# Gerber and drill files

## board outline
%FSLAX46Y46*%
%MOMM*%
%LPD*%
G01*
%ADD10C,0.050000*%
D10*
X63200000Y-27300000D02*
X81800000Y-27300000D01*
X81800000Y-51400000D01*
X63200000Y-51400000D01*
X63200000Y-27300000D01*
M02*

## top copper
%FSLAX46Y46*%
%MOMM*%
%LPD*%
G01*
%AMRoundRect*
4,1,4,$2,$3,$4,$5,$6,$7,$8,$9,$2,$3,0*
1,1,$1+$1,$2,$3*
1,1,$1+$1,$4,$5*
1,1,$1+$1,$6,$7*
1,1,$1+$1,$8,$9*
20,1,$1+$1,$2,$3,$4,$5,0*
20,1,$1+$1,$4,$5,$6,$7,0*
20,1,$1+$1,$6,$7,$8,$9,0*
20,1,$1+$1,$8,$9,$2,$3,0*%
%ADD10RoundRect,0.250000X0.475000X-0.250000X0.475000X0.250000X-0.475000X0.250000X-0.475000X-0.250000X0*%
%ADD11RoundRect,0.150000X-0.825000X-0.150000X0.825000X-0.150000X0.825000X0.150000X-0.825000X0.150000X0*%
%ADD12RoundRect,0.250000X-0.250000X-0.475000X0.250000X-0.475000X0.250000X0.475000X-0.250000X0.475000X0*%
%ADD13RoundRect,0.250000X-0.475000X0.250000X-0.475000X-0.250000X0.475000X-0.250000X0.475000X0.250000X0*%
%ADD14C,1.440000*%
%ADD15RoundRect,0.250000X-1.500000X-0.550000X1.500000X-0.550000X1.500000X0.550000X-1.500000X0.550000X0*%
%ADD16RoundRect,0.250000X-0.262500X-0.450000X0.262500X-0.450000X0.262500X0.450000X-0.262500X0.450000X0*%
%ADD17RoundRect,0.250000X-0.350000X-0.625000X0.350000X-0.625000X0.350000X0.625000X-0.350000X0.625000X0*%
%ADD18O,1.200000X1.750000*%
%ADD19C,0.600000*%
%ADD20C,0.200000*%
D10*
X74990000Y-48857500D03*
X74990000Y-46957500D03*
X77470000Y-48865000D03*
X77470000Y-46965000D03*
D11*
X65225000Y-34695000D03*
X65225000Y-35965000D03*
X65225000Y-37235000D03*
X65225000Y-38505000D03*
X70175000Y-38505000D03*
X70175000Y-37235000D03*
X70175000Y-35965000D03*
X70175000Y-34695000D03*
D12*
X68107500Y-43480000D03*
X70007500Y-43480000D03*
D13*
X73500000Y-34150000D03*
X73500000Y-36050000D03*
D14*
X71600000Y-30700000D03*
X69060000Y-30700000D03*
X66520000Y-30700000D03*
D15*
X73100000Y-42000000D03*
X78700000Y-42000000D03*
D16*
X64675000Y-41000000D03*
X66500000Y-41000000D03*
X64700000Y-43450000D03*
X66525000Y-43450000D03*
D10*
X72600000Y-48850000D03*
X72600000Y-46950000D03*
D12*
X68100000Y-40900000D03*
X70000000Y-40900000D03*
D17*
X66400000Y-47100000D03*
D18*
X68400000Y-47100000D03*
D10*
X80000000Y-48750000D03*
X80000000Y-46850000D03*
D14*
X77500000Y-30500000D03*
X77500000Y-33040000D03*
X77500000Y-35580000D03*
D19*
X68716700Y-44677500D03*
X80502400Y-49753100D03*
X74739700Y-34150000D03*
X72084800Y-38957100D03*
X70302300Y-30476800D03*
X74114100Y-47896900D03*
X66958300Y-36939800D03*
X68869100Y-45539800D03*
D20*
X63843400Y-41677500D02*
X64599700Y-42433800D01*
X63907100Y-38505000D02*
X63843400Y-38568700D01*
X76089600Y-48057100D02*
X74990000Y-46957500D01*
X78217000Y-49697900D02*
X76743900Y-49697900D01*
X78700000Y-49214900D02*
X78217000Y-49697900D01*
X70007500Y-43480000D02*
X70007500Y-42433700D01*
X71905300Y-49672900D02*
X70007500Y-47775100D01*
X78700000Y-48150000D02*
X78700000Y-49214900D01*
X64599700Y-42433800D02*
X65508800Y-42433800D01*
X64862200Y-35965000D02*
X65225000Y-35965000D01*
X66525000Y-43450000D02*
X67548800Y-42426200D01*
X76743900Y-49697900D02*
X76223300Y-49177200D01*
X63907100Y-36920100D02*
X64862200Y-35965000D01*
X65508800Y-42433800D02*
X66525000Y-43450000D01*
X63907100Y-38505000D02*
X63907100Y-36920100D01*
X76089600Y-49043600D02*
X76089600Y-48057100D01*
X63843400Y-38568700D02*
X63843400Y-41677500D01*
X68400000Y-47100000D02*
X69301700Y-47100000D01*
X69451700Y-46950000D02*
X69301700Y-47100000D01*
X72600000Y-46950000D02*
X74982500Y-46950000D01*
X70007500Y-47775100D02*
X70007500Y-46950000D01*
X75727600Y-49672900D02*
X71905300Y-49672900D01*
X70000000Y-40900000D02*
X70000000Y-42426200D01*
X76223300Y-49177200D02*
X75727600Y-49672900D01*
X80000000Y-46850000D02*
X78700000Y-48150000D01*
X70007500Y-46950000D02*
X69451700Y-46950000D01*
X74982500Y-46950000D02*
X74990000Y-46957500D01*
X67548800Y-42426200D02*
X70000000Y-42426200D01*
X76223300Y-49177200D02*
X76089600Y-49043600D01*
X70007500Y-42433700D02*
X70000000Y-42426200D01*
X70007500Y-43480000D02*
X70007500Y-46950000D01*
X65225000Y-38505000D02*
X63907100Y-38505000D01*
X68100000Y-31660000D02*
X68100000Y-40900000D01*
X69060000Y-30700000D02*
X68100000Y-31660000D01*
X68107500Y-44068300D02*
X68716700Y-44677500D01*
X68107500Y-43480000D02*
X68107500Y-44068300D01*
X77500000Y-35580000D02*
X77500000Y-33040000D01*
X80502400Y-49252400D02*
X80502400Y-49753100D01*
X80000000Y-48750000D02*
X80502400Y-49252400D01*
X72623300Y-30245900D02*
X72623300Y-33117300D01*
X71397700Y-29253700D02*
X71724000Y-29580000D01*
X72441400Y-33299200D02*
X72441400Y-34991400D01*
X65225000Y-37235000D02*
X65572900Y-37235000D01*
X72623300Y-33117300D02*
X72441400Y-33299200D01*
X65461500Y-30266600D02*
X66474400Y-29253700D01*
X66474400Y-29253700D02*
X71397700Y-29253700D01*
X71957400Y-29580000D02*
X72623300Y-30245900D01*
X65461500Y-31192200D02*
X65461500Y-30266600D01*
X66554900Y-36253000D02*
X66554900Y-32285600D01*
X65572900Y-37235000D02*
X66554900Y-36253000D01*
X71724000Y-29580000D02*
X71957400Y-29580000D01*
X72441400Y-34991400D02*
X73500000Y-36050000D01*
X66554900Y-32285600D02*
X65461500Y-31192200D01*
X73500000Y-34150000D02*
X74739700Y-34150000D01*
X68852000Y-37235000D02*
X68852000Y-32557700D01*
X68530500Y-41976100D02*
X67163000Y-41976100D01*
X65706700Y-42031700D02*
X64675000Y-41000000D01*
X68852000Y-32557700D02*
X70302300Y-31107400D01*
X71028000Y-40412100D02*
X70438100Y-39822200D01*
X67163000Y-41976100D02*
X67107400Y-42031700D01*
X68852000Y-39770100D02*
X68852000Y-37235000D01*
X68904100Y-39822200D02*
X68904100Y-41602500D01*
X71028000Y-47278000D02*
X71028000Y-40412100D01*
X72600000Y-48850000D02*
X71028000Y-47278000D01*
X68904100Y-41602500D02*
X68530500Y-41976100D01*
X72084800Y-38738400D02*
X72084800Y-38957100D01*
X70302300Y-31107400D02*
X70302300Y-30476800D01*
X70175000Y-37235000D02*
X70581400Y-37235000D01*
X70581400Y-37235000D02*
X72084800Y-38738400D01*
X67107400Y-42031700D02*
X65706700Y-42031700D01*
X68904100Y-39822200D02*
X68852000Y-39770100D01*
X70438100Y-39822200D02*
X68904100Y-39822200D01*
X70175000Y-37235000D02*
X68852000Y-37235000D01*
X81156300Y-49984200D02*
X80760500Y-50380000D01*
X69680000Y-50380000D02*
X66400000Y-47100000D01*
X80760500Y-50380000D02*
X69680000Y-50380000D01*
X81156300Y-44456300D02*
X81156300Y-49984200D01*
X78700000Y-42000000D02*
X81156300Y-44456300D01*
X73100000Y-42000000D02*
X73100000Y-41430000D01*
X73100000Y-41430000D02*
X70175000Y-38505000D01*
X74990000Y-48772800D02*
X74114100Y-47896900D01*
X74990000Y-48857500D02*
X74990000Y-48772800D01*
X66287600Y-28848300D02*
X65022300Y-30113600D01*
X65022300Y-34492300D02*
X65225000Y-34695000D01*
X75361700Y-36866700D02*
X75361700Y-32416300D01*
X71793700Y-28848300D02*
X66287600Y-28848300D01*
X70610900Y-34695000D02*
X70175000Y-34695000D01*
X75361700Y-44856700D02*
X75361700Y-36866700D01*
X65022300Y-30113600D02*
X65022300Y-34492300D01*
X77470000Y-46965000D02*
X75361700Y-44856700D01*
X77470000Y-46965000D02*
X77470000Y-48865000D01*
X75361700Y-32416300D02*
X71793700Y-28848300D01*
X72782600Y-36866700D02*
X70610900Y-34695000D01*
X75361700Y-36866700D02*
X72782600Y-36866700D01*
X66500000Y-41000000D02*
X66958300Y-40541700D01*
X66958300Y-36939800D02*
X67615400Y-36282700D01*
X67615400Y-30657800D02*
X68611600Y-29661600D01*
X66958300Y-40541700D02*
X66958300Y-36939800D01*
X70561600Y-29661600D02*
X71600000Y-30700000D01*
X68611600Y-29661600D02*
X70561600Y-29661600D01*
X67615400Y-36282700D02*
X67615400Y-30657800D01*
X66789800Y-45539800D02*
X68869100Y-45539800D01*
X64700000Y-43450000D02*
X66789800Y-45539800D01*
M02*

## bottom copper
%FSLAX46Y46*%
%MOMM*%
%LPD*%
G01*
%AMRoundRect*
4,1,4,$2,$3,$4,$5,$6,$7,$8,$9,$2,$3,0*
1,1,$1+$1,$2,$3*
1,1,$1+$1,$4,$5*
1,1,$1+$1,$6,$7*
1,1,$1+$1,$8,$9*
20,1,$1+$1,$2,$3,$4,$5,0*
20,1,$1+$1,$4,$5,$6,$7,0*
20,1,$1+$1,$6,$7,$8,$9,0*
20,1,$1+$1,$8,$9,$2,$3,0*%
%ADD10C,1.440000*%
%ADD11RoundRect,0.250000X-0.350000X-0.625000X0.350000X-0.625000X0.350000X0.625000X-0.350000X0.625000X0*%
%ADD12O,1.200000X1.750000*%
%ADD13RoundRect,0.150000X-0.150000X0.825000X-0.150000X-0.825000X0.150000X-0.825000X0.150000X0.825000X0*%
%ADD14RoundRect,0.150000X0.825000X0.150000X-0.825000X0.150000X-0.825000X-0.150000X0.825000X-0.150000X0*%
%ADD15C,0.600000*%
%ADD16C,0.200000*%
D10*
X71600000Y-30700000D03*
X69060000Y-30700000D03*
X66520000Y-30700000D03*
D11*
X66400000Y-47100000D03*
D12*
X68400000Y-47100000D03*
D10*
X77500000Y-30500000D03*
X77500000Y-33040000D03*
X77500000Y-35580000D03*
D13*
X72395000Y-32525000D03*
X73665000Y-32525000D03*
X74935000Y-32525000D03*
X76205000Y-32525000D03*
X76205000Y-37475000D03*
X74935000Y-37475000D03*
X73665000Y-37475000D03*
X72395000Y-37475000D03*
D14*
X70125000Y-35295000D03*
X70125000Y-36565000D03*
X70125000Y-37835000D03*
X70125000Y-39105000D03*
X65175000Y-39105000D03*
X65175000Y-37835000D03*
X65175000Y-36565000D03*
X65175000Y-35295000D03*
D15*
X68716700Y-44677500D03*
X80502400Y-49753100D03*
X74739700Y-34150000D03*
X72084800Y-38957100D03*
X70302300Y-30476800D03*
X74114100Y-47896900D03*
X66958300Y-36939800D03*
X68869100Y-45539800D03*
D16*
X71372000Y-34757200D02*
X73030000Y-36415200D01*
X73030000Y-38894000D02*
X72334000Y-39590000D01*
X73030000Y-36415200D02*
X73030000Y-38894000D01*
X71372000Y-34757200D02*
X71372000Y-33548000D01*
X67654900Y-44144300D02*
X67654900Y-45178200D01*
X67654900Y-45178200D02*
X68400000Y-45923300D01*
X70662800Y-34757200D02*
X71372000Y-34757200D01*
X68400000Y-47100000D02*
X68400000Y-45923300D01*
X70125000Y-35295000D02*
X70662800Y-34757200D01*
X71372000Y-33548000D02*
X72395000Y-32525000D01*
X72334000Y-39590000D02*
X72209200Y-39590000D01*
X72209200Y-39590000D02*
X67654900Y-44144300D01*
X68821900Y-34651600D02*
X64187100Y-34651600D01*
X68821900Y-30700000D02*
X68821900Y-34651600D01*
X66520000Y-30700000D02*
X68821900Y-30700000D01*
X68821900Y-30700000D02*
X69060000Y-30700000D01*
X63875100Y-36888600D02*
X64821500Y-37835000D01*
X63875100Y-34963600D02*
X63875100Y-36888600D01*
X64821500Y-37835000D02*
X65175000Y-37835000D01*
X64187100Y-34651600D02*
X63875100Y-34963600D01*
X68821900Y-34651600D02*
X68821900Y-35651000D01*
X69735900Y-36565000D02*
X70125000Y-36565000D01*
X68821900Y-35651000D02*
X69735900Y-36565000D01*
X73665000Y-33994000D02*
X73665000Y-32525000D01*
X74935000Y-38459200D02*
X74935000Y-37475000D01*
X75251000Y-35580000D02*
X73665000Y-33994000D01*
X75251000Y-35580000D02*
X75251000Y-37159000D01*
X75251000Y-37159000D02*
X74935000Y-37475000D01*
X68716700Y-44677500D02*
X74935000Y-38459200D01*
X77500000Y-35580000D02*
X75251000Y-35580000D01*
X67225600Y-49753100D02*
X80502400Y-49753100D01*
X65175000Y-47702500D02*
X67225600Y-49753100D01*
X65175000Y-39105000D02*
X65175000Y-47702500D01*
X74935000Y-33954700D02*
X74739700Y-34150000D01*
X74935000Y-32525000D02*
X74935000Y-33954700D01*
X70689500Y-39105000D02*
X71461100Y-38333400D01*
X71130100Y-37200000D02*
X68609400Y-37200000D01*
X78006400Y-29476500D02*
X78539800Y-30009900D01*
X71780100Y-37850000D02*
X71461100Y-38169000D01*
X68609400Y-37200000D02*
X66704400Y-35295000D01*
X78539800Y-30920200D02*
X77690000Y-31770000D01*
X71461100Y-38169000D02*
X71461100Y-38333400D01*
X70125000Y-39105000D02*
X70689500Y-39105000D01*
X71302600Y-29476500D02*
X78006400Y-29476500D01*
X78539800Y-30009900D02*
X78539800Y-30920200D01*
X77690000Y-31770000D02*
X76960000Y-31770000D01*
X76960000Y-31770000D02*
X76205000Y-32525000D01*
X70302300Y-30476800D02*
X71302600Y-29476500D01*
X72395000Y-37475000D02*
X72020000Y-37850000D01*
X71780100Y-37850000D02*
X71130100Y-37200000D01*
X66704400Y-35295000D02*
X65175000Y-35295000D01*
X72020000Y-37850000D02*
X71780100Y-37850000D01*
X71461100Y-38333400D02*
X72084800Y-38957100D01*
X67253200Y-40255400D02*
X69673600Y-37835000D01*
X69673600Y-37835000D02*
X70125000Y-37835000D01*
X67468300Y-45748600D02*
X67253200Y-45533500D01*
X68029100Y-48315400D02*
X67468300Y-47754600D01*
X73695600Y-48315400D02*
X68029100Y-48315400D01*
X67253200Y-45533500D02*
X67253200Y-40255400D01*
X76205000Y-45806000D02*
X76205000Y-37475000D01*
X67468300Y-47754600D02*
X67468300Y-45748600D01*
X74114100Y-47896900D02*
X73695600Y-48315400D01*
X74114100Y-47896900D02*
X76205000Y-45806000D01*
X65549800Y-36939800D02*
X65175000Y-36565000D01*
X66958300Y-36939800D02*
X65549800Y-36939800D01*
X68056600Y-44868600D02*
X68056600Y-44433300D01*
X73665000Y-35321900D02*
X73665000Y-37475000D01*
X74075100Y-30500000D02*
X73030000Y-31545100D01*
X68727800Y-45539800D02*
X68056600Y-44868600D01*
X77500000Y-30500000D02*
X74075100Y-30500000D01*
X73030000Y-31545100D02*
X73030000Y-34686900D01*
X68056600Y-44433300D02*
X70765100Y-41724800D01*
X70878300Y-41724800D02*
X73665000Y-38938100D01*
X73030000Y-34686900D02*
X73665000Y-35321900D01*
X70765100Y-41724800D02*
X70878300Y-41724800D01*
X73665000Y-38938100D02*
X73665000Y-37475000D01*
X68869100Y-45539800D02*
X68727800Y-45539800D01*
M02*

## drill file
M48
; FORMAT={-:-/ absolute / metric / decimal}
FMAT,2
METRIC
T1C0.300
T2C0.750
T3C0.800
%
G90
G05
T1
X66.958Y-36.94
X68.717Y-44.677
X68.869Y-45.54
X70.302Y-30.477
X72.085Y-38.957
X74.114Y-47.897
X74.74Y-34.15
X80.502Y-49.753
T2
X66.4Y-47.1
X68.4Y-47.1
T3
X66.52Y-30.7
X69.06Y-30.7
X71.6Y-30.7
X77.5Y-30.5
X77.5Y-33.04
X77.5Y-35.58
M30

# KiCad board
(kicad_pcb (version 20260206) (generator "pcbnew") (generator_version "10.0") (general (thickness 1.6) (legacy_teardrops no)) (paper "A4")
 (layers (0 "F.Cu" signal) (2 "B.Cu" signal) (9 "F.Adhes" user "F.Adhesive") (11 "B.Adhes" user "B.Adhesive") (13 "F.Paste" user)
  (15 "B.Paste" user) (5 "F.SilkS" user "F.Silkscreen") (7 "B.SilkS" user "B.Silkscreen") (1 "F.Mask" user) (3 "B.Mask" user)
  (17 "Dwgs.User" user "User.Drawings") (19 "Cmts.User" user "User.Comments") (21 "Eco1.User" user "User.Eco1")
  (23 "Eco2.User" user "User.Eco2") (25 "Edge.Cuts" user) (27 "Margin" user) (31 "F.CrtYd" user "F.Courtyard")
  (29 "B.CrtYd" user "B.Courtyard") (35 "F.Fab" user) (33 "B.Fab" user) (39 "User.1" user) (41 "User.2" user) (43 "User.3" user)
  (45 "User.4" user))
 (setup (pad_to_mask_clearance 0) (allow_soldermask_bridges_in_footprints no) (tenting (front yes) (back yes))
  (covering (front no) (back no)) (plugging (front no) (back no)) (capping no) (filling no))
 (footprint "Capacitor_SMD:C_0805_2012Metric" (layer "F.Cu") (at 74.99 47.9075 90)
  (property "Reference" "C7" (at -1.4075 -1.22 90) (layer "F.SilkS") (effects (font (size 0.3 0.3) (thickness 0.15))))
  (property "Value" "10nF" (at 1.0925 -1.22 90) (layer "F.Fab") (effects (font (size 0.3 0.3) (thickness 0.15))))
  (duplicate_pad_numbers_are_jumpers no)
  (pad "1" smd roundrect (at -0.95 0 90) (size 1 1.45) (layers "F.Cu" "F.Mask" "F.Paste") (roundrect_rratio 0.25) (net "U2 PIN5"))
  (pad "2" smd roundrect (at 0.95 0 90) (size 1 1.45) (layers "F.Cu" "F.Mask" "F.Paste") (roundrect_rratio 0.25) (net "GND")))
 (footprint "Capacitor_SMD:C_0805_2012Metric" (layer "F.Cu") (at 77.47 47.915 90)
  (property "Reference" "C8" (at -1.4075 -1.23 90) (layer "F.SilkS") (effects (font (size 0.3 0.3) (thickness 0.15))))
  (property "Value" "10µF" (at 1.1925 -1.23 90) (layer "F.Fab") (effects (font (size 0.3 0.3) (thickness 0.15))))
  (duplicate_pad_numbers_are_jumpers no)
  (pad "1" smd roundrect (at -0.95 0 90) (size 1 1.45) (layers "F.Cu" "F.Mask" "F.Paste") (roundrect_rratio 0.25) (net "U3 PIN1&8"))
  (pad "2" smd roundrect (at 0.95 0 90) (size 1 1.45) (layers "F.Cu" "F.Mask" "F.Paste") (roundrect_rratio 0.25) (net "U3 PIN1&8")))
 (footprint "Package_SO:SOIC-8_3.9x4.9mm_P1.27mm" (layer "F.Cu") (at 67.7 36.6)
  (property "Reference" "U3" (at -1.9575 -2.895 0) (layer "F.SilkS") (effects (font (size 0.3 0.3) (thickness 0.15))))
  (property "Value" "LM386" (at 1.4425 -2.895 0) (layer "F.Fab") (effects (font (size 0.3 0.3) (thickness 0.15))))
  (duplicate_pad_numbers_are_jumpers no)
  (pad "1" smd roundrect (at -2.475 -1.905) (size 1.95 0.6) (layers "F.Cu" "F.Mask" "F.Paste") (roundrect_rratio 0.25) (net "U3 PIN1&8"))
  (pad "2" smd roundrect (at -2.475 -0.635) (size 1.95 0.6) (layers "F.Cu" "F.Mask" "F.Paste") (roundrect_rratio 0.25) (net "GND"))
  (pad "3" smd roundrect (at -2.475 0.635) (size 1.95 0.6) (layers "F.Cu" "F.Mask" "F.Paste") (roundrect_rratio 0.25) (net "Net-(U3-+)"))
  (pad "4" smd roundrect (at -2.475 1.905) (size 1.95 0.6) (layers "F.Cu" "F.Mask" "F.Paste") (roundrect_rratio 0.25) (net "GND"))
  (pad "5" smd roundrect (at 2.475 1.905) (size 1.95 0.6) (layers "F.Cu" "F.Mask" "F.Paste") (roundrect_rratio 0.25) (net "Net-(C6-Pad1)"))
  (pad "6" smd roundrect (at 2.475 0.635) (size 1.95 0.6) (layers "F.Cu" "F.Mask" "F.Paste") (roundrect_rratio 0.25) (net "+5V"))
  (pad "7" smd roundrect (at 2.475 -0.635) (size 1.95 0.6) (layers "F.Cu" "F.Mask" "F.Paste") (roundrect_rratio 0.25)
   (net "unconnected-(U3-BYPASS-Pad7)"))
  (pad "8" smd roundrect (at 2.475 -1.905) (size 1.95 0.6) (layers "F.Cu" "F.Mask" "F.Paste") (roundrect_rratio 0.25) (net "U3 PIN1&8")))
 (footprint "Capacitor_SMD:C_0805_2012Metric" (layer "F.Cu") (at 69.0575 43.48)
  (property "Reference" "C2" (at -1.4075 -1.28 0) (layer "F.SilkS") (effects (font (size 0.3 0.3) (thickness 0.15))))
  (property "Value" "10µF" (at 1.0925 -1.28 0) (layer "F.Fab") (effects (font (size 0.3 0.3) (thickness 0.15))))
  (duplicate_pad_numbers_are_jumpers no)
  (pad "1" smd roundrect (at -0.95 0) (size 1 1.45) (layers "F.Cu" "F.Mask" "F.Paste") (roundrect_rratio 0.25) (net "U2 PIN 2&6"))
  (pad "2" smd roundrect (at 0.95 0) (size 1 1.45) (layers "F.Cu" "F.Mask" "F.Paste") (roundrect_rratio 0.25) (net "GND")))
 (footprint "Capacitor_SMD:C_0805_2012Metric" (layer "F.Cu") (at 73.5 35.1 -90)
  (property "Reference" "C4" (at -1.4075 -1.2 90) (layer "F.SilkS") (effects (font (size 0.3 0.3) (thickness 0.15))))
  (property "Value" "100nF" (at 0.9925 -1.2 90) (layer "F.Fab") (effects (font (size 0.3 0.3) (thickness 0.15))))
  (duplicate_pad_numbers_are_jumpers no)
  (pad "1" smd roundrect (at -0.95 0 270) (size 1 1.45) (layers "F.Cu" "F.Mask" "F.Paste") (roundrect_rratio 0.25) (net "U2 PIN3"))
  (pad "2" smd roundrect (at 0.95 0 270) (size 1 1.45) (layers "F.Cu" "F.Mask" "F.Paste") (roundrect_rratio 0.25) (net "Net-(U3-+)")))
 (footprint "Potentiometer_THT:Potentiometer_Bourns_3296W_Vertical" (layer "F.Cu") (at 71.6 30.7)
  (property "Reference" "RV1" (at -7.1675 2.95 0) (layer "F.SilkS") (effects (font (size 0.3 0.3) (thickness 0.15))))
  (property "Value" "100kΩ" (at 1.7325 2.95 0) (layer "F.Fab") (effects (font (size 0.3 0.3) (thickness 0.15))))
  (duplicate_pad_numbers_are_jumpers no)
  (pad "1" thru_hole circle (at 0 0) (size 1.44 1.44) (drill 0.8) (layers "*.Cu" "*.Mask") (remove_unused_layers no) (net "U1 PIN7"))
  (pad "2" thru_hole circle (at -2.54 0) (size 1.44 1.44) (drill 0.8) (layers "*.Cu" "*.Mask") (remove_unused_layers no) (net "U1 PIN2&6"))
  (pad "3" thru_hole circle (at -5.08 0) (size 1.44 1.44) (drill 0.8) (layers "*.Cu" "*.Mask") (remove_unused_layers no) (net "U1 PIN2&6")))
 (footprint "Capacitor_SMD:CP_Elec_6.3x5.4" (layer "F.Cu") (at 75.9 42)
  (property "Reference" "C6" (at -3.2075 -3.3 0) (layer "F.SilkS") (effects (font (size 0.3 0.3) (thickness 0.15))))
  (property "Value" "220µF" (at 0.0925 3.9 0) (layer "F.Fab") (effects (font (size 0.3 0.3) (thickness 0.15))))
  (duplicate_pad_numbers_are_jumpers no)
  (pad "1" smd roundrect (at -2.8 0) (size 3.5 1.6) (layers "F.Cu" "F.Mask" "F.Paste") (roundrect_rratio 0.15625) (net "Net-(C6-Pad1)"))
  (pad "2" smd roundrect (at 2.8 0) (size 3.5 1.6) (layers "F.Cu" "F.Mask" "F.Paste") (roundrect_rratio 0.15625) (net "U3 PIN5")))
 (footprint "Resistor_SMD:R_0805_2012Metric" (layer "F.Cu") (at 65.5875 41)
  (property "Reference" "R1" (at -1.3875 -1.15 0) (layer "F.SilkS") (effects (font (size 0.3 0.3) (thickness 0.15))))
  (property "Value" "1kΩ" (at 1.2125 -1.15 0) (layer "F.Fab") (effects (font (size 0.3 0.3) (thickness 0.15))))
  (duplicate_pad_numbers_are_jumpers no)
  (pad "1" smd roundrect (at -0.9125 0) (size 1.025 1.4) (layers "F.Cu" "F.Mask" "F.Paste") (roundrect_rratio 0.243902) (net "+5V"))
  (pad "2" smd roundrect (at 0.9125 0) (size 1.025 1.4) (layers "F.Cu" "F.Mask" "F.Paste") (roundrect_rratio 0.243902) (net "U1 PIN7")))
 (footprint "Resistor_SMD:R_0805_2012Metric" (layer "F.Cu") (at 65.6125 43.45)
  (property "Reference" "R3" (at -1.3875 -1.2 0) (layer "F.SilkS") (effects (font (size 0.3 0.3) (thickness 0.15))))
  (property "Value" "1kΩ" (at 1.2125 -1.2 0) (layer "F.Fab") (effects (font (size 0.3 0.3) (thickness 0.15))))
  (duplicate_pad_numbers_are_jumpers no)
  (pad "1" smd roundrect (at -0.9125 0) (size 1.025 1.4) (layers "F.Cu" "F.Mask" "F.Paste") (roundrect_rratio 0.243902) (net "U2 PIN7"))
  (pad "2" smd roundrect (at 0.9125 0) (size 1.025 1.4) (layers "F.Cu" "F.Mask" "F.Paste") (roundrect_rratio 0.243902) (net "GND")))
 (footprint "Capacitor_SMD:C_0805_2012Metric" (layer "F.Cu") (at 72.6 47.9 90)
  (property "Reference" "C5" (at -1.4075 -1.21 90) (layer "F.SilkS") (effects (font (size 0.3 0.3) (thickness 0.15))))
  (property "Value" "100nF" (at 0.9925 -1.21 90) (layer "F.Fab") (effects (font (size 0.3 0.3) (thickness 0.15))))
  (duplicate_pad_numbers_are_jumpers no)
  (pad "1" smd roundrect (at -0.95 0 90) (size 1 1.45) (layers "F.Cu" "F.Mask" "F.Paste") (roundrect_rratio 0.25) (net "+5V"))
  (pad "2" smd roundrect (at 0.95 0 90) (size 1 1.45) (layers "F.Cu" "F.Mask" "F.Paste") (roundrect_rratio 0.25) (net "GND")))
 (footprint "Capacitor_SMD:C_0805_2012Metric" (layer "F.Cu") (at 69.05 40.9)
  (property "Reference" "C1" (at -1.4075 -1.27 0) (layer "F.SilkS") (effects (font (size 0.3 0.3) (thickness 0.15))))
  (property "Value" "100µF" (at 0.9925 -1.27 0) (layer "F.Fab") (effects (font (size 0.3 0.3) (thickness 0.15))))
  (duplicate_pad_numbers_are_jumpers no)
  (pad "1" smd roundrect (at -0.95 0) (size 1 1.45) (layers "F.Cu" "F.Mask" "F.Paste") (roundrect_rratio 0.25) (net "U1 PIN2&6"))
  (pad "2" smd roundrect (at 0.95 0) (size 1 1.45) (layers "F.Cu" "F.Mask" "F.Paste") (roundrect_rratio 0.25) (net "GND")))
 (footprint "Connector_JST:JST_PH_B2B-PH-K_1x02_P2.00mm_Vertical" (layer "F.Cu") (at 66.4 47.1)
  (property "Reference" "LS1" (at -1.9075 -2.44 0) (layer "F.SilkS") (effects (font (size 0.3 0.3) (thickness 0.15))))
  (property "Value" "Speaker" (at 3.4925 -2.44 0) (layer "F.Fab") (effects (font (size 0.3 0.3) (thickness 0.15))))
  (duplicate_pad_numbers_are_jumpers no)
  (pad "1" thru_hole roundrect (at 0 0) (size 1.2 1.75) (drill 0.75) (layers "*.Cu" "*.Mask") (remove_unused_layers no)
   (roundrect_rratio 0.208333) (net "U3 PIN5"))
  (pad "2" thru_hole oval (at 2 0) (size 1.2 1.75) (drill 0.75) (layers "*.Cu" "*.Mask") (remove_unused_layers no) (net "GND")))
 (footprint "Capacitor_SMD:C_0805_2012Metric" (layer "F.Cu") (at 80 47.8 90)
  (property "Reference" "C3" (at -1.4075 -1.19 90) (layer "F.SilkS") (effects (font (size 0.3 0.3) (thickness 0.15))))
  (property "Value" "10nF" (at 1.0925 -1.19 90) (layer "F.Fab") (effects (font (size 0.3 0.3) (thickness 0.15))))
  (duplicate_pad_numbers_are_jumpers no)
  (pad "1" smd roundrect (at -0.95 0 90) (size 1 1.45) (layers "F.Cu" "F.Mask" "F.Paste") (roundrect_rratio 0.25) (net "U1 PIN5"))
  (pad "2" smd roundrect (at 0.95 0 90) (size 1 1.45) (layers "F.Cu" "F.Mask" "F.Paste") (roundrect_rratio 0.25) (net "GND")))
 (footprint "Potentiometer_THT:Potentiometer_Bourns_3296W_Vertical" (layer "F.Cu") (at 77.5 30.5 90)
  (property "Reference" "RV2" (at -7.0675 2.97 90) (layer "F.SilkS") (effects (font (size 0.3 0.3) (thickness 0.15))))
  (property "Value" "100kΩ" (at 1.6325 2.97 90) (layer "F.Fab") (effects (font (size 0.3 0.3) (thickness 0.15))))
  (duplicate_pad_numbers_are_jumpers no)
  (pad "1" thru_hole circle (at 0 0 90) (size 1.44 1.44) (drill 0.8) (layers "*.Cu" "*.Mask") (remove_unused_layers no) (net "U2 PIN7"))
  (pad "2" thru_hole circle (at -2.54 0 90) (size 1.44 1.44) (drill 0.8) (layers "*.Cu" "*.Mask") (remove_unused_layers no)
   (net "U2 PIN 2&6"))
  (pad "3" thru_hole circle (at -5.08 0 90) (size 1.44 1.44) (drill 0.8) (layers "*.Cu" "*.Mask") (remove_unused_layers no)
   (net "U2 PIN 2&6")))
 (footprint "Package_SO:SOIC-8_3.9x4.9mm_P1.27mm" (layer "B.Cu") (at 74.3 35 -90)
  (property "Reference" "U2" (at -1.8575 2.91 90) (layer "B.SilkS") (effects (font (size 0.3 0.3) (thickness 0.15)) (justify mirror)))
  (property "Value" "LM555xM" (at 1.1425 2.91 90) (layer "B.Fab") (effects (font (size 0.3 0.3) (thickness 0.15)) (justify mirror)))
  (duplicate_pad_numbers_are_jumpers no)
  (pad "1" smd roundrect (at -2.475 1.905 270) (size 1.95 0.6) (layers "B.Cu" "B.Mask" "B.Paste") (roundrect_rratio 0.25) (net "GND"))
  (pad "2" smd roundrect (at -2.475 0.635 270) (size 1.95 0.6) (layers "B.Cu" "B.Mask" "B.Paste") (roundrect_rratio 0.25) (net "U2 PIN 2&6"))
  (pad "3" smd roundrect (at -2.475 -0.635 270) (size 1.95 0.6) (layers "B.Cu" "B.Mask" "B.Paste") (roundrect_rratio 0.25) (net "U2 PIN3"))
  (pad "4" smd roundrect (at -2.475 -1.905 270) (size 1.95 0.6) (layers "B.Cu" "B.Mask" "B.Paste") (roundrect_rratio 0.25) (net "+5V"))
  (pad "5" smd roundrect (at 2.475 -1.905 270) (size 1.95 0.6) (layers "B.Cu" "B.Mask" "B.Paste") (roundrect_rratio 0.25) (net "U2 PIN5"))
  (pad "6" smd roundrect (at 2.475 -0.635 270) (size 1.95 0.6) (layers "B.Cu" "B.Mask" "B.Paste") (roundrect_rratio 0.25) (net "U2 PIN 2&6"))
  (pad "7" smd roundrect (at 2.475 0.635 270) (size 1.95 0.6) (layers "B.Cu" "B.Mask" "B.Paste") (roundrect_rratio 0.25) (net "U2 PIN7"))
  (pad "8" smd roundrect (at 2.475 1.905 270) (size 1.95 0.6) (layers "B.Cu" "B.Mask" "B.Paste") (roundrect_rratio 0.25) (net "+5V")))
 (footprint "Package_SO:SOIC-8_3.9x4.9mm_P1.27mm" (layer "B.Cu") (at 67.65 37.2 180)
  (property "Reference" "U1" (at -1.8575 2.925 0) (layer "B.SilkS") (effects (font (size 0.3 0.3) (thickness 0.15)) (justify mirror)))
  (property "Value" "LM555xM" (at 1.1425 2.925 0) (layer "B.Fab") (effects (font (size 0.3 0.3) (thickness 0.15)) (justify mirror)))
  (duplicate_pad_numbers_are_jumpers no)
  (pad "1" smd roundrect (at -2.475 1.905 180) (size 1.95 0.6) (layers "B.Cu" "B.Mask" "B.Paste") (roundrect_rratio 0.25) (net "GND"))
  (pad "2" smd roundrect (at -2.475 0.635 180) (size 1.95 0.6) (layers "B.Cu" "B.Mask" "B.Paste") (roundrect_rratio 0.25) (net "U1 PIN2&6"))
  (pad "3" smd roundrect (at -2.475 -0.635 180) (size 1.95 0.6) (layers "B.Cu" "B.Mask" "B.Paste") (roundrect_rratio 0.25) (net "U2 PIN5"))
  (pad "4" smd roundrect (at -2.475 -1.905 180) (size 1.95 0.6) (layers "B.Cu" "B.Mask" "B.Paste") (roundrect_rratio 0.25) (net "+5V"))
  (pad "5" smd roundrect (at 2.475 -1.905 180) (size 1.95 0.6) (layers "B.Cu" "B.Mask" "B.Paste") (roundrect_rratio 0.25) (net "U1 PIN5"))
  (pad "6" smd roundrect (at 2.475 -0.635 180) (size 1.95 0.6) (layers "B.Cu" "B.Mask" "B.Paste") (roundrect_rratio 0.25) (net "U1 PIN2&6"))
  (pad "7" smd roundrect (at 2.475 0.635 180) (size 1.95 0.6) (layers "B.Cu" "B.Mask" "B.Paste") (roundrect_rratio 0.25) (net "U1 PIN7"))
  (pad "8" smd roundrect (at 2.475 1.905 180) (size 1.95 0.6) (layers "B.Cu" "B.Mask" "B.Paste") (roundrect_rratio 0.25) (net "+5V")))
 (gr_rect (start 63.2 27.3) (end 81.8 51.4) (stroke (width 0.05) (type default)) (fill no) (layer "Edge.Cuts"))
 (segment (start 63.8434 41.6775) (end 64.5997 42.4338) (width 0.2) (layer "F.Cu") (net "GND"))
 (segment (start 63.9071 38.505) (end 63.8434 38.5687) (width 0.2) (layer "F.Cu") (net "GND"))
 (segment (start 76.0896 48.0571) (end 74.99 46.9575) (width 0.2) (layer "F.Cu") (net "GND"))
 (segment (start 78.217 49.6979) (end 76.7439 49.6979) (width 0.2) (layer "F.Cu") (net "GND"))
 (segment (start 78.7 49.2149) (end 78.217 49.6979) (width 0.2) (layer "F.Cu") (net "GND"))
 (segment (start 70.0075 43.48) (end 70.0075 42.4337) (width 0.2) (layer "F.Cu") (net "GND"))
 (segment (start 71.9053 49.6729) (end 70.0075 47.7751) (width 0.2) (layer "F.Cu") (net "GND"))
 (segment (start 78.7 48.15) (end 78.7 49.2149) (width 0.2) (layer "F.Cu") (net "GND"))
 (segment (start 64.5997 42.4338) (end 65.5088 42.4338) (width 0.2) (layer "F.Cu") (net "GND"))
 (segment (start 64.8622 35.965) (end 65.225 35.965) (width 0.2) (layer "F.Cu") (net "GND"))
 (segment (start 66.525 43.45) (end 67.5488 42.4262) (width 0.2) (layer "F.Cu") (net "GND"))
 (segment (start 76.7439 49.6979) (end 76.2233 49.1772) (width 0.2) (layer "F.Cu") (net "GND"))
 (segment (start 63.9071 36.9201) (end 64.8622 35.965) (width 0.2) (layer "F.Cu") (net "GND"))
 (segment (start 65.5088 42.4338) (end 66.525 43.45) (width 0.2) (layer "F.Cu") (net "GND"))
 (segment (start 63.9071 38.505) (end 63.9071 36.9201) (width 0.2) (layer "F.Cu") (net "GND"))
 (segment (start 76.0896 49.0436) (end 76.0896 48.0571) (width 0.2) (layer "F.Cu") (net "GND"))
 (segment (start 63.8434 38.5687) (end 63.8434 41.6775) (width 0.2) (layer "F.Cu") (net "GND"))
 (segment (start 68.4 47.1) (end 69.3017 47.1) (width 0.2) (layer "F.Cu") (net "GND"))
 (segment (start 69.4517 46.95) (end 69.3017 47.1) (width 0.2) (layer "F.Cu") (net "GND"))
 (segment (start 72.6 46.95) (end 74.9825 46.95) (width 0.2) (layer "F.Cu") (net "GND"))
 (segment (start 70.0075 47.7751) (end 70.0075 46.95) (width 0.2) (layer "F.Cu") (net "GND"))
 (segment (start 75.7276 49.6729) (end 71.9053 49.6729) (width 0.2) (layer "F.Cu") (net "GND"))
 (segment (start 70 40.9) (end 70 42.4262) (width 0.2) (layer "F.Cu") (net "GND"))
 (segment (start 76.2233 49.1772) (end 75.7276 49.6729) (width 0.2) (layer "F.Cu") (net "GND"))
 (segment (start 80 46.85) (end 78.7 48.15) (width 0.2) (layer "F.Cu") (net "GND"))
 (segment (start 70.0075 46.95) (end 69.4517 46.95) (width 0.2) (layer "F.Cu") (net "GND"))
 (segment (start 74.9825 46.95) (end 74.99 46.9575) (width 0.2) (layer "F.Cu") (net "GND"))
 (segment (start 67.5488 42.4262) (end 70 42.4262) (width 0.2) (layer "F.Cu") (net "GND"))
 (segment (start 76.2233 49.1772) (end 76.0896 49.0436) (width 0.2) (layer "F.Cu") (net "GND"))
 (segment (start 70.0075 42.4337) (end 70 42.4262) (width 0.2) (layer "F.Cu") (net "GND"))
 (segment (start 70.0075 43.48) (end 70.0075 46.95) (width 0.2) (layer "F.Cu") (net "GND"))
 (segment (start 65.225 38.505) (end 63.9071 38.505) (width 0.2) (layer "F.Cu") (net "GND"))
 (segment (start 71.372 34.7572) (end 73.03 36.4152) (width 0.2) (layer "B.Cu") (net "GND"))
 (segment (start 73.03 38.894) (end 72.334 39.59) (width 0.2) (layer "B.Cu") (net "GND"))
 (segment (start 73.03 36.4152) (end 73.03 38.894) (width 0.2) (layer "B.Cu") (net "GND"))
 (segment (start 71.372 34.7572) (end 71.372 33.548) (width 0.2) (layer "B.Cu") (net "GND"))
 (segment (start 67.6549 44.1443) (end 67.6549 45.1782) (width 0.2) (layer "B.Cu") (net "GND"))
 (segment (start 67.6549 45.1782) (end 68.4 45.9233) (width 0.2) (layer "B.Cu") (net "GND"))
 (segment (start 70.6628 34.7572) (end 71.372 34.7572) (width 0.2) (layer "B.Cu") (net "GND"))
 (segment (start 68.4 47.1) (end 68.4 45.9233) (width 0.2) (layer "B.Cu") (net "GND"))
 (segment (start 70.125 35.295) (end 70.6628 34.7572) (width 0.2) (layer "B.Cu") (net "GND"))
 (segment (start 71.372 33.548) (end 72.395 32.525) (width 0.2) (layer "B.Cu") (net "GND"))
 (segment (start 72.334 39.59) (end 72.2092 39.59) (width 0.2) (layer "B.Cu") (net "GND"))
 (segment (start 72.2092 39.59) (end 67.6549 44.1443) (width 0.2) (layer "B.Cu") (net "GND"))
 (segment (start 68.1 31.66) (end 68.1 40.9) (width 0.2) (layer "F.Cu") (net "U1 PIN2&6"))
 (segment (start 69.06 30.7) (end 68.1 31.66) (width 0.2) (layer "F.Cu") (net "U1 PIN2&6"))
 (segment (start 68.8219 34.6516) (end 64.1871 34.6516) (width 0.2) (layer "B.Cu") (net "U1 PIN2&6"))
 (segment (start 68.8219 30.7) (end 68.8219 34.6516) (width 0.2) (layer "B.Cu") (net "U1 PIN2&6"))
 (segment (start 66.52 30.7) (end 68.8219 30.7) (width 0.2) (layer "B.Cu") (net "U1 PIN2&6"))
 (segment (start 68.8219 30.7) (end 69.06 30.7) (width 0.2) (layer "B.Cu") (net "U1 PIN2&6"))
 (segment (start 63.8751 36.8886) (end 64.8215 37.835) (width 0.2) (layer "B.Cu") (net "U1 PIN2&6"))
 (segment (start 63.8751 34.9636) (end 63.8751 36.8886) (width 0.2) (layer "B.Cu") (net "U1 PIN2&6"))
 (segment (start 64.8215 37.835) (end 65.175 37.835) (width 0.2) (layer "B.Cu") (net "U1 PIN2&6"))
 (segment (start 64.1871 34.6516) (end 63.8751 34.9636) (width 0.2) (layer "B.Cu") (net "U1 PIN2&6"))
 (segment (start 68.8219 34.6516) (end 68.8219 35.651) (width 0.2) (layer "B.Cu") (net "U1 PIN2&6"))
 (segment (start 69.7359 36.565) (end 70.125 36.565) (width 0.2) (layer "B.Cu") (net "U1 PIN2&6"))
 (segment (start 68.8219 35.651) (end 69.7359 36.565) (width 0.2) (layer "B.Cu") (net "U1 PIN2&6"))
 (segment (start 68.1075 44.0683) (end 68.7167 44.6775) (width 0.2) (layer "F.Cu") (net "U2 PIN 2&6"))
 (segment (start 68.1075 43.48) (end 68.1075 44.0683) (width 0.2) (layer "F.Cu") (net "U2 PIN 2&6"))
 (segment (start 77.5 35.58) (end 77.5 33.04) (width 0.2) (layer "F.Cu") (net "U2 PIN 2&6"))
 (via (at 68.7167 44.6775) (size 0.6) (drill 0.3) (layers "F.Cu" "B.Cu") (capping no) (covering (front no) (back no))
  (plugging (front no) (back no)) (filling no) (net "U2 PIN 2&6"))
 (segment (start 73.665 33.994) (end 73.665 32.525) (width 0.2) (layer "B.Cu") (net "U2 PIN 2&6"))
 (segment (start 74.935 38.4592) (end 74.935 37.475) (width 0.2) (layer "B.Cu") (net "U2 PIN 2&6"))
 (segment (start 75.251 35.58) (end 73.665 33.994) (width 0.2) (layer "B.Cu") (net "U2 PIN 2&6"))
 (segment (start 75.251 35.58) (end 75.251 37.159) (width 0.2) (layer "B.Cu") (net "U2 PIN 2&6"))
 (segment (start 75.251 37.159) (end 74.935 37.475) (width 0.2) (layer "B.Cu") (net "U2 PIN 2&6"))
 (segment (start 68.7167 44.6775) (end 74.935 38.4592) (width 0.2) (layer "B.Cu") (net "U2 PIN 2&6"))
 (segment (start 77.5 35.58) (end 75.251 35.58) (width 0.2) (layer "B.Cu") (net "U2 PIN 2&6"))
 (segment (start 80.5024 49.2524) (end 80.5024 49.7531) (width 0.2) (layer "F.Cu") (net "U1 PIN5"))
 (segment (start 80 48.75) (end 80.5024 49.2524) (width 0.2) (layer "F.Cu") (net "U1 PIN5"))
 (via (at 80.5024 49.7531) (size 0.6) (drill 0.3) (layers "F.Cu" "B.Cu") (capping no) (covering (front no) (back no))
  (plugging (front no) (back no)) (filling no) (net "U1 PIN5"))
 (segment (start 67.2256 49.7531) (end 80.5024 49.7531) (width 0.2) (layer "B.Cu") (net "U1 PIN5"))
 (segment (start 65.175 47.7025) (end 67.2256 49.7531) (width 0.2) (layer "B.Cu") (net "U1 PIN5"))
 (segment (start 65.175 39.105) (end 65.175 47.7025) (width 0.2) (layer "B.Cu") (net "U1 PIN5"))
 (segment (start 72.6233 30.2459) (end 72.6233 33.1173) (width 0.2) (layer "F.Cu") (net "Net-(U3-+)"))
 (segment (start 71.3977 29.2537) (end 71.724 29.58) (width 0.2) (layer "F.Cu") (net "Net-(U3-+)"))
 (segment (start 72.4414 33.2992) (end 72.4414 34.9914) (width 0.2) (layer "F.Cu") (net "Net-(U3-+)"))
 (segment (start 65.225 37.235) (end 65.5729 37.235) (width 0.2) (layer "F.Cu") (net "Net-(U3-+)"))
 (segment (start 72.6233 33.1173) (end 72.4414 33.2992) (width 0.2) (layer "F.Cu") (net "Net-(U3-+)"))
 (segment (start 65.4615 30.2666) (end 66.4744 29.2537) (width 0.2) (layer "F.Cu") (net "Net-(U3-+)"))
 (segment (start 66.4744 29.2537) (end 71.3977 29.2537) (width 0.2) (layer "F.Cu") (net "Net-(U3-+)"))
 (segment (start 71.9574 29.58) (end 72.6233 30.2459) (width 0.2) (layer "F.Cu") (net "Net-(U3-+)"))
 (segment (start 65.4615 31.1922) (end 65.4615 30.2666) (width 0.2) (layer "F.Cu") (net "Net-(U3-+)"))
 (segment (start 66.5549 36.253) (end 66.5549 32.2856) (width 0.2) (layer "F.Cu") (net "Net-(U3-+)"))
 (segment (start 65.5729 37.235) (end 66.5549 36.253) (width 0.2) (layer "F.Cu") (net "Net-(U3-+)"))
 (segment (start 71.724 29.58) (end 71.9574 29.58) (width 0.2) (layer "F.Cu") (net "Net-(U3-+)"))
 (segment (start 72.4414 34.9914) (end 73.5 36.05) (width 0.2) (layer "F.Cu") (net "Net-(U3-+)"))
 (segment (start 66.5549 32.2856) (end 65.4615 31.1922) (width 0.2) (layer "F.Cu") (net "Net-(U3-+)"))
 (segment (start 73.5 34.15) (end 74.7397 34.15) (width 0.2) (layer "F.Cu") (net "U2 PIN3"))
 (via (at 74.7397 34.15) (size 0.6) (drill 0.3) (layers "F.Cu" "B.Cu") (capping no) (covering (front no) (back no))
  (plugging (front no) (back no)) (filling no) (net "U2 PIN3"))
 (segment (start 74.935 33.9547) (end 74.7397 34.15) (width 0.2) (layer "B.Cu") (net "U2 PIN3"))
 (segment (start 74.935 32.525) (end 74.935 33.9547) (width 0.2) (layer "B.Cu") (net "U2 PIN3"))
 (segment (start 68.852 37.235) (end 68.852 32.5577) (width 0.2) (layer "F.Cu") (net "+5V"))
 (segment (start 68.5305 41.9761) (end 67.163 41.9761) (width 0.2) (layer "F.Cu") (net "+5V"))
 (segment (start 65.7067 42.0317) (end 64.675 41) (width 0.2) (layer "F.Cu") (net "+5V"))
 (segment (start 68.852 32.5577) (end 70.3023 31.1074) (width 0.2) (layer "F.Cu") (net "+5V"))
 (segment (start 71.028 40.4121) (end 70.4381 39.8222) (width 0.2) (layer "F.Cu") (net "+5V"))
 (segment (start 67.163 41.9761) (end 67.1074 42.0317) (width 0.2) (layer "F.Cu") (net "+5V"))
 (segment (start 68.852 39.7701) (end 68.852 37.235) (width 0.2) (layer "F.Cu") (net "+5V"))
 (segment (start 68.9041 39.8222) (end 68.9041 41.6025) (width 0.2) (layer "F.Cu") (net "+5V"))
 (segment (start 71.028 47.278) (end 71.028 40.4121) (width 0.2) (layer "F.Cu") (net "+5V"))
 (segment (start 72.6 48.85) (end 71.028 47.278) (width 0.2) (layer "F.Cu") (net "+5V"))
 (segment (start 68.9041 41.6025) (end 68.5305 41.9761) (width 0.2) (layer "F.Cu") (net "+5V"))
 (segment (start 72.0848 38.7384) (end 72.0848 38.9571) (width 0.2) (layer "F.Cu") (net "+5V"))
 (segment (start 70.3023 31.1074) (end 70.3023 30.4768) (width 0.2) (layer "F.Cu") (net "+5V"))
 (segment (start 70.175 37.235) (end 70.5814 37.235) (width 0.2) (layer "F.Cu") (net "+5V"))
 (segment (start 70.5814 37.235) (end 72.0848 38.7384) (width 0.2) (layer "F.Cu") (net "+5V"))
 (segment (start 67.1074 42.0317) (end 65.7067 42.0317) (width 0.2) (layer "F.Cu") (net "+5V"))
 (segment (start 68.9041 39.8222) (end 68.852 39.7701) (width 0.2) (layer "F.Cu") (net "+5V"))
 (segment (start 70.4381 39.8222) (end 68.9041 39.8222) (width 0.2) (layer "F.Cu") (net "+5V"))
 (segment (start 70.175 37.235) (end 68.852 37.235) (width 0.2) (layer "F.Cu") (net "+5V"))
 (via (at 72.0848 38.9571) (size 0.6) (drill 0.3) (layers "F.Cu" "B.Cu") (capping no) (covering (front no) (back no))
  (plugging (front no) (back no)) (filling no) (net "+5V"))
 (via (at 70.3023 30.4768) (size 0.6) (drill 0.3) (layers "F.Cu" "B.Cu") (capping no) (covering (front no) (back no))
  (plugging (front no) (back no)) (filling no) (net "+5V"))
 (segment (start 70.6895 39.105) (end 71.4611 38.3334) (width 0.2) (layer "B.Cu") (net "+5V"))
 (segment (start 71.1301 37.2) (end 68.6094 37.2) (width 0.2) (layer "B.Cu") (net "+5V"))
 (segment (start 78.0064 29.4765) (end 78.5398 30.0099) (width 0.2) (layer "B.Cu") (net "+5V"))
 (segment (start 71.7801 37.85) (end 71.4611 38.169) (width 0.2) (layer "B.Cu") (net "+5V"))
 (segment (start 68.6094 37.2) (end 66.7044 35.295) (width 0.2) (layer "B.Cu") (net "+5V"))
 (segment (start 78.5398 30.9202) (end 77.69 31.77) (width 0.2) (layer "B.Cu") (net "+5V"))
 (segment (start 71.4611 38.169) (end 71.4611 38.3334) (width 0.2) (layer "B.Cu") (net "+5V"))
 (segment (start 70.125 39.105) (end 70.6895 39.105) (width 0.2) (layer "B.Cu") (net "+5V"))
 (segment (start 71.3026 29.4765) (end 78.0064 29.4765) (width 0.2) (layer "B.Cu") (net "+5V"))
 (segment (start 78.5398 30.0099) (end 78.5398 30.9202) (width 0.2) (layer "B.Cu") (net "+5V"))
 (segment (start 77.69 31.77) (end 76.96 31.77) (width 0.2) (layer "B.Cu") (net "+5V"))
 (segment (start 76.96 31.77) (end 76.205 32.525) (width 0.2) (layer "B.Cu") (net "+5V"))
 (segment (start 70.3023 30.4768) (end 71.3026 29.4765) (width 0.2) (layer "B.Cu") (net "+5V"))
 (segment (start 72.395 37.475) (end 72.02 37.85) (width 0.2) (layer "B.Cu") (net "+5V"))
 (segment (start 71.7801 37.85) (end 71.1301 37.2) (width 0.2) (layer "B.Cu") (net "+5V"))
 (segment (start 66.7044 35.295) (end 65.175 35.295) (width 0.2) (layer "B.Cu") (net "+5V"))
 (segment (start 72.02 37.85) (end 71.7801 37.85) (width 0.2) (layer "B.Cu") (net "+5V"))
 (segment (start 71.4611 38.3334) (end 72.0848 38.9571) (width 0.2) (layer "B.Cu") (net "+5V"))
 (segment (start 81.1563 49.9842) (end 80.7605 50.38) (width 0.2) (layer "F.Cu") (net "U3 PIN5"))
 (segment (start 69.68 50.38) (end 66.4 47.1) (width 0.2) (layer "F.Cu") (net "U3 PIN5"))
 (segment (start 80.7605 50.38) (end 69.68 50.38) (width 0.2) (layer "F.Cu") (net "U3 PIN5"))
 (segment (start 81.1563 44.4563) (end 81.1563 49.9842) (width 0.2) (layer "F.Cu") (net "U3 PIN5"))
 (segment (start 78.7 42) (end 81.1563 44.4563) (width 0.2) (layer "F.Cu") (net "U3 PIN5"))
 (segment (start 73.1 42) (end 73.1 41.43) (width 0.2) (layer "F.Cu") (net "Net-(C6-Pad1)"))
 (segment (start 73.1 41.43) (end 70.175 38.505) (width 0.2) (layer "F.Cu") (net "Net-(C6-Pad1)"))
 (segment (start 74.99 48.7728) (end 74.1141 47.8969) (width 0.2) (layer "F.Cu") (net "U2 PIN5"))
 (segment (start 74.99 48.8575) (end 74.99 48.7728) (width 0.2) (layer "F.Cu") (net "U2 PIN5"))
 (via (at 74.1141 47.8969) (size 0.6) (drill 0.3) (layers "F.Cu" "B.Cu") (capping no) (covering (front no) (back no))
  (plugging (front no) (back no)) (filling no) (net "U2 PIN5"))
 (segment (start 67.2532 40.2554) (end 69.6736 37.835) (width 0.2) (layer "B.Cu") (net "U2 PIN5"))
 (segment (start 69.6736 37.835) (end 70.125 37.835) (width 0.2) (layer "B.Cu") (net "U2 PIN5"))
 (segment (start 67.4683 45.7486) (end 67.2532 45.5335) (width 0.2) (layer "B.Cu") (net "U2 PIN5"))
 (segment (start 68.0291 48.3154) (end 67.4683 47.7546) (width 0.2) (layer "B.Cu") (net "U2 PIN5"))
 (segment (start 73.6956 48.3154) (end 68.0291 48.3154) (width 0.2) (layer "B.Cu") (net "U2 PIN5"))
 (segment (start 67.2532 45.5335) (end 67.2532 40.2554) (width 0.2) (layer "B.Cu") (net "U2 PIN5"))
 (segment (start 76.205 45.806) (end 76.205 37.475) (width 0.2) (layer "B.Cu") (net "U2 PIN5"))
 (segment (start 67.4683 47.7546) (end 67.4683 45.7486) (width 0.2) (layer "B.Cu") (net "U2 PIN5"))
 (segment (start 74.1141 47.8969) (end 73.6956 48.3154) (width 0.2) (layer "B.Cu") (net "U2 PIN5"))
 (segment (start 74.1141 47.8969) (end 76.205 45.806) (width 0.2) (layer "B.Cu") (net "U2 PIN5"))
 (segment (start 66.2876 28.8483) (end 65.0223 30.1136) (width 0.2) (layer "F.Cu") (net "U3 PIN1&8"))
 (segment (start 65.0223 34.4923) (end 65.225 34.695) (width 0.2) (layer "F.Cu") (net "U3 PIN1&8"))
 (segment (start 75.3617 36.8667) (end 75.3617 32.4163) (width 0.2) (layer "F.Cu") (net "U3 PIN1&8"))
 (segment (start 71.7937 28.8483) (end 66.2876 28.8483) (width 0.2) (layer "F.Cu") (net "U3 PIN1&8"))
 (segment (start 70.6109 34.695) (end 70.175 34.695) (width 0.2) (layer "F.Cu") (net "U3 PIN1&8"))
 (segment (start 75.3617 44.8567) (end 75.3617 36.8667) (width 0.2) (layer "F.Cu") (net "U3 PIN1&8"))
 (segment (start 65.0223 30.1136) (end 65.0223 34.4923) (width 0.2) (layer "F.Cu") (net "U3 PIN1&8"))
 (segment (start 77.47 46.965) (end 75.3617 44.8567) (width 0.2) (layer "F.Cu") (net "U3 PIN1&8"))
 (segment (start 77.47 46.965) (end 77.47 48.865) (width 0.2) (layer "F.Cu") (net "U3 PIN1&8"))
 (segment (start 75.3617 32.4163) (end 71.7937 28.8483) (width 0.2) (layer "F.Cu") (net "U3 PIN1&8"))
 (segment (start 72.7826 36.8667) (end 70.6109 34.695) (width 0.2) (layer "F.Cu") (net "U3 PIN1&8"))
 (segment (start 75.3617 36.8667) (end 72.7826 36.8667) (width 0.2) (layer "F.Cu") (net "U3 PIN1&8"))
 (segment (start 66.5 41) (end 66.9583 40.5417) (width 0.2) (layer "F.Cu") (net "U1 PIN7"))
 (segment (start 66.9583 36.9398) (end 67.6154 36.2827) (width 0.2) (layer "F.Cu") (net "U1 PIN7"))
 (segment (start 67.6154 30.6578) (end 68.6116 29.6616) (width 0.2) (layer "F.Cu") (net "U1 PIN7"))
 (segment (start 66.9583 40.5417) (end 66.9583 36.9398) (width 0.2) (layer "F.Cu") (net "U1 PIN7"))
 (segment (start 70.5616 29.6616) (end 71.6 30.7) (width 0.2) (layer "F.Cu") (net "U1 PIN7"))
 (segment (start 68.6116 29.6616) (end 70.5616 29.6616) (width 0.2) (layer "F.Cu") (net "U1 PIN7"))
 (segment (start 67.6154 36.2827) (end 67.6154 30.6578) (width 0.2) (layer "F.Cu") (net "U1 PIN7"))
 (via (at 66.9583 36.9398) (size 0.6) (drill 0.3) (layers "F.Cu" "B.Cu") (capping no) (covering (front no) (back no))
  (plugging (front no) (back no)) (filling no) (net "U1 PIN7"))
 (segment (start 65.5498 36.9398) (end 65.175 36.565) (width 0.2) (layer "B.Cu") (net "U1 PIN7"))
 (segment (start 66.9583 36.9398) (end 65.5498 36.9398) (width 0.2) (layer "B.Cu") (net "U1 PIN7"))
 (segment (start 66.7898 45.5398) (end 68.8691 45.5398) (width 0.2) (layer "F.Cu") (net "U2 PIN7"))
 (segment (start 64.7 43.45) (end 66.7898 45.5398) (width 0.2) (layer "F.Cu") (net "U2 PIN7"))
 (via (at 68.8691 45.5398) (size 0.6) (drill 0.3) (layers "F.Cu" "B.Cu") (capping no) (covering (front no) (back no))
  (plugging (front no) (back no)) (filling no) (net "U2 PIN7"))
 (segment (start 68.0566 44.8686) (end 68.0566 44.4333) (width 0.2) (layer "B.Cu") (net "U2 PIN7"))
 (segment (start 73.665 35.3219) (end 73.665 37.475) (width 0.2) (layer "B.Cu") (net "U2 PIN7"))
 (segment (start 74.0751 30.5) (end 73.03 31.5451) (width 0.2) (layer "B.Cu") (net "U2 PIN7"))
 (segment (start 68.7278 45.5398) (end 68.0566 44.8686) (width 0.2) (layer "B.Cu") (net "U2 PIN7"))
 (segment (start 77.5 30.5) (end 74.0751 30.5) (width 0.2) (layer "B.Cu") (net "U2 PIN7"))
 (segment (start 73.03 31.5451) (end 73.03 34.6869) (width 0.2) (layer "B.Cu") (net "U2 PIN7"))
 (segment (start 68.0566 44.4333) (end 70.7651 41.7248) (width 0.2) (layer "B.Cu") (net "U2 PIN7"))
 (segment (start 70.8783 41.7248) (end 73.665 38.9381) (width 0.2) (layer "B.Cu") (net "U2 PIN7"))
 (segment (start 73.03 34.6869) (end 73.665 35.3219) (width 0.2) (layer "B.Cu") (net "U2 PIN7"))
 (segment (start 70.7651 41.7248) (end 70.8783 41.7248) (width 0.2) (layer "B.Cu") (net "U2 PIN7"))
 (segment (start 73.665 38.9381) (end 73.665 37.475) (width 0.2) (layer "B.Cu") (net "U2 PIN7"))
 (segment (start 68.8691 45.5398) (end 68.7278 45.5398) (width 0.2) (layer "B.Cu") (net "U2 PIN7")))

